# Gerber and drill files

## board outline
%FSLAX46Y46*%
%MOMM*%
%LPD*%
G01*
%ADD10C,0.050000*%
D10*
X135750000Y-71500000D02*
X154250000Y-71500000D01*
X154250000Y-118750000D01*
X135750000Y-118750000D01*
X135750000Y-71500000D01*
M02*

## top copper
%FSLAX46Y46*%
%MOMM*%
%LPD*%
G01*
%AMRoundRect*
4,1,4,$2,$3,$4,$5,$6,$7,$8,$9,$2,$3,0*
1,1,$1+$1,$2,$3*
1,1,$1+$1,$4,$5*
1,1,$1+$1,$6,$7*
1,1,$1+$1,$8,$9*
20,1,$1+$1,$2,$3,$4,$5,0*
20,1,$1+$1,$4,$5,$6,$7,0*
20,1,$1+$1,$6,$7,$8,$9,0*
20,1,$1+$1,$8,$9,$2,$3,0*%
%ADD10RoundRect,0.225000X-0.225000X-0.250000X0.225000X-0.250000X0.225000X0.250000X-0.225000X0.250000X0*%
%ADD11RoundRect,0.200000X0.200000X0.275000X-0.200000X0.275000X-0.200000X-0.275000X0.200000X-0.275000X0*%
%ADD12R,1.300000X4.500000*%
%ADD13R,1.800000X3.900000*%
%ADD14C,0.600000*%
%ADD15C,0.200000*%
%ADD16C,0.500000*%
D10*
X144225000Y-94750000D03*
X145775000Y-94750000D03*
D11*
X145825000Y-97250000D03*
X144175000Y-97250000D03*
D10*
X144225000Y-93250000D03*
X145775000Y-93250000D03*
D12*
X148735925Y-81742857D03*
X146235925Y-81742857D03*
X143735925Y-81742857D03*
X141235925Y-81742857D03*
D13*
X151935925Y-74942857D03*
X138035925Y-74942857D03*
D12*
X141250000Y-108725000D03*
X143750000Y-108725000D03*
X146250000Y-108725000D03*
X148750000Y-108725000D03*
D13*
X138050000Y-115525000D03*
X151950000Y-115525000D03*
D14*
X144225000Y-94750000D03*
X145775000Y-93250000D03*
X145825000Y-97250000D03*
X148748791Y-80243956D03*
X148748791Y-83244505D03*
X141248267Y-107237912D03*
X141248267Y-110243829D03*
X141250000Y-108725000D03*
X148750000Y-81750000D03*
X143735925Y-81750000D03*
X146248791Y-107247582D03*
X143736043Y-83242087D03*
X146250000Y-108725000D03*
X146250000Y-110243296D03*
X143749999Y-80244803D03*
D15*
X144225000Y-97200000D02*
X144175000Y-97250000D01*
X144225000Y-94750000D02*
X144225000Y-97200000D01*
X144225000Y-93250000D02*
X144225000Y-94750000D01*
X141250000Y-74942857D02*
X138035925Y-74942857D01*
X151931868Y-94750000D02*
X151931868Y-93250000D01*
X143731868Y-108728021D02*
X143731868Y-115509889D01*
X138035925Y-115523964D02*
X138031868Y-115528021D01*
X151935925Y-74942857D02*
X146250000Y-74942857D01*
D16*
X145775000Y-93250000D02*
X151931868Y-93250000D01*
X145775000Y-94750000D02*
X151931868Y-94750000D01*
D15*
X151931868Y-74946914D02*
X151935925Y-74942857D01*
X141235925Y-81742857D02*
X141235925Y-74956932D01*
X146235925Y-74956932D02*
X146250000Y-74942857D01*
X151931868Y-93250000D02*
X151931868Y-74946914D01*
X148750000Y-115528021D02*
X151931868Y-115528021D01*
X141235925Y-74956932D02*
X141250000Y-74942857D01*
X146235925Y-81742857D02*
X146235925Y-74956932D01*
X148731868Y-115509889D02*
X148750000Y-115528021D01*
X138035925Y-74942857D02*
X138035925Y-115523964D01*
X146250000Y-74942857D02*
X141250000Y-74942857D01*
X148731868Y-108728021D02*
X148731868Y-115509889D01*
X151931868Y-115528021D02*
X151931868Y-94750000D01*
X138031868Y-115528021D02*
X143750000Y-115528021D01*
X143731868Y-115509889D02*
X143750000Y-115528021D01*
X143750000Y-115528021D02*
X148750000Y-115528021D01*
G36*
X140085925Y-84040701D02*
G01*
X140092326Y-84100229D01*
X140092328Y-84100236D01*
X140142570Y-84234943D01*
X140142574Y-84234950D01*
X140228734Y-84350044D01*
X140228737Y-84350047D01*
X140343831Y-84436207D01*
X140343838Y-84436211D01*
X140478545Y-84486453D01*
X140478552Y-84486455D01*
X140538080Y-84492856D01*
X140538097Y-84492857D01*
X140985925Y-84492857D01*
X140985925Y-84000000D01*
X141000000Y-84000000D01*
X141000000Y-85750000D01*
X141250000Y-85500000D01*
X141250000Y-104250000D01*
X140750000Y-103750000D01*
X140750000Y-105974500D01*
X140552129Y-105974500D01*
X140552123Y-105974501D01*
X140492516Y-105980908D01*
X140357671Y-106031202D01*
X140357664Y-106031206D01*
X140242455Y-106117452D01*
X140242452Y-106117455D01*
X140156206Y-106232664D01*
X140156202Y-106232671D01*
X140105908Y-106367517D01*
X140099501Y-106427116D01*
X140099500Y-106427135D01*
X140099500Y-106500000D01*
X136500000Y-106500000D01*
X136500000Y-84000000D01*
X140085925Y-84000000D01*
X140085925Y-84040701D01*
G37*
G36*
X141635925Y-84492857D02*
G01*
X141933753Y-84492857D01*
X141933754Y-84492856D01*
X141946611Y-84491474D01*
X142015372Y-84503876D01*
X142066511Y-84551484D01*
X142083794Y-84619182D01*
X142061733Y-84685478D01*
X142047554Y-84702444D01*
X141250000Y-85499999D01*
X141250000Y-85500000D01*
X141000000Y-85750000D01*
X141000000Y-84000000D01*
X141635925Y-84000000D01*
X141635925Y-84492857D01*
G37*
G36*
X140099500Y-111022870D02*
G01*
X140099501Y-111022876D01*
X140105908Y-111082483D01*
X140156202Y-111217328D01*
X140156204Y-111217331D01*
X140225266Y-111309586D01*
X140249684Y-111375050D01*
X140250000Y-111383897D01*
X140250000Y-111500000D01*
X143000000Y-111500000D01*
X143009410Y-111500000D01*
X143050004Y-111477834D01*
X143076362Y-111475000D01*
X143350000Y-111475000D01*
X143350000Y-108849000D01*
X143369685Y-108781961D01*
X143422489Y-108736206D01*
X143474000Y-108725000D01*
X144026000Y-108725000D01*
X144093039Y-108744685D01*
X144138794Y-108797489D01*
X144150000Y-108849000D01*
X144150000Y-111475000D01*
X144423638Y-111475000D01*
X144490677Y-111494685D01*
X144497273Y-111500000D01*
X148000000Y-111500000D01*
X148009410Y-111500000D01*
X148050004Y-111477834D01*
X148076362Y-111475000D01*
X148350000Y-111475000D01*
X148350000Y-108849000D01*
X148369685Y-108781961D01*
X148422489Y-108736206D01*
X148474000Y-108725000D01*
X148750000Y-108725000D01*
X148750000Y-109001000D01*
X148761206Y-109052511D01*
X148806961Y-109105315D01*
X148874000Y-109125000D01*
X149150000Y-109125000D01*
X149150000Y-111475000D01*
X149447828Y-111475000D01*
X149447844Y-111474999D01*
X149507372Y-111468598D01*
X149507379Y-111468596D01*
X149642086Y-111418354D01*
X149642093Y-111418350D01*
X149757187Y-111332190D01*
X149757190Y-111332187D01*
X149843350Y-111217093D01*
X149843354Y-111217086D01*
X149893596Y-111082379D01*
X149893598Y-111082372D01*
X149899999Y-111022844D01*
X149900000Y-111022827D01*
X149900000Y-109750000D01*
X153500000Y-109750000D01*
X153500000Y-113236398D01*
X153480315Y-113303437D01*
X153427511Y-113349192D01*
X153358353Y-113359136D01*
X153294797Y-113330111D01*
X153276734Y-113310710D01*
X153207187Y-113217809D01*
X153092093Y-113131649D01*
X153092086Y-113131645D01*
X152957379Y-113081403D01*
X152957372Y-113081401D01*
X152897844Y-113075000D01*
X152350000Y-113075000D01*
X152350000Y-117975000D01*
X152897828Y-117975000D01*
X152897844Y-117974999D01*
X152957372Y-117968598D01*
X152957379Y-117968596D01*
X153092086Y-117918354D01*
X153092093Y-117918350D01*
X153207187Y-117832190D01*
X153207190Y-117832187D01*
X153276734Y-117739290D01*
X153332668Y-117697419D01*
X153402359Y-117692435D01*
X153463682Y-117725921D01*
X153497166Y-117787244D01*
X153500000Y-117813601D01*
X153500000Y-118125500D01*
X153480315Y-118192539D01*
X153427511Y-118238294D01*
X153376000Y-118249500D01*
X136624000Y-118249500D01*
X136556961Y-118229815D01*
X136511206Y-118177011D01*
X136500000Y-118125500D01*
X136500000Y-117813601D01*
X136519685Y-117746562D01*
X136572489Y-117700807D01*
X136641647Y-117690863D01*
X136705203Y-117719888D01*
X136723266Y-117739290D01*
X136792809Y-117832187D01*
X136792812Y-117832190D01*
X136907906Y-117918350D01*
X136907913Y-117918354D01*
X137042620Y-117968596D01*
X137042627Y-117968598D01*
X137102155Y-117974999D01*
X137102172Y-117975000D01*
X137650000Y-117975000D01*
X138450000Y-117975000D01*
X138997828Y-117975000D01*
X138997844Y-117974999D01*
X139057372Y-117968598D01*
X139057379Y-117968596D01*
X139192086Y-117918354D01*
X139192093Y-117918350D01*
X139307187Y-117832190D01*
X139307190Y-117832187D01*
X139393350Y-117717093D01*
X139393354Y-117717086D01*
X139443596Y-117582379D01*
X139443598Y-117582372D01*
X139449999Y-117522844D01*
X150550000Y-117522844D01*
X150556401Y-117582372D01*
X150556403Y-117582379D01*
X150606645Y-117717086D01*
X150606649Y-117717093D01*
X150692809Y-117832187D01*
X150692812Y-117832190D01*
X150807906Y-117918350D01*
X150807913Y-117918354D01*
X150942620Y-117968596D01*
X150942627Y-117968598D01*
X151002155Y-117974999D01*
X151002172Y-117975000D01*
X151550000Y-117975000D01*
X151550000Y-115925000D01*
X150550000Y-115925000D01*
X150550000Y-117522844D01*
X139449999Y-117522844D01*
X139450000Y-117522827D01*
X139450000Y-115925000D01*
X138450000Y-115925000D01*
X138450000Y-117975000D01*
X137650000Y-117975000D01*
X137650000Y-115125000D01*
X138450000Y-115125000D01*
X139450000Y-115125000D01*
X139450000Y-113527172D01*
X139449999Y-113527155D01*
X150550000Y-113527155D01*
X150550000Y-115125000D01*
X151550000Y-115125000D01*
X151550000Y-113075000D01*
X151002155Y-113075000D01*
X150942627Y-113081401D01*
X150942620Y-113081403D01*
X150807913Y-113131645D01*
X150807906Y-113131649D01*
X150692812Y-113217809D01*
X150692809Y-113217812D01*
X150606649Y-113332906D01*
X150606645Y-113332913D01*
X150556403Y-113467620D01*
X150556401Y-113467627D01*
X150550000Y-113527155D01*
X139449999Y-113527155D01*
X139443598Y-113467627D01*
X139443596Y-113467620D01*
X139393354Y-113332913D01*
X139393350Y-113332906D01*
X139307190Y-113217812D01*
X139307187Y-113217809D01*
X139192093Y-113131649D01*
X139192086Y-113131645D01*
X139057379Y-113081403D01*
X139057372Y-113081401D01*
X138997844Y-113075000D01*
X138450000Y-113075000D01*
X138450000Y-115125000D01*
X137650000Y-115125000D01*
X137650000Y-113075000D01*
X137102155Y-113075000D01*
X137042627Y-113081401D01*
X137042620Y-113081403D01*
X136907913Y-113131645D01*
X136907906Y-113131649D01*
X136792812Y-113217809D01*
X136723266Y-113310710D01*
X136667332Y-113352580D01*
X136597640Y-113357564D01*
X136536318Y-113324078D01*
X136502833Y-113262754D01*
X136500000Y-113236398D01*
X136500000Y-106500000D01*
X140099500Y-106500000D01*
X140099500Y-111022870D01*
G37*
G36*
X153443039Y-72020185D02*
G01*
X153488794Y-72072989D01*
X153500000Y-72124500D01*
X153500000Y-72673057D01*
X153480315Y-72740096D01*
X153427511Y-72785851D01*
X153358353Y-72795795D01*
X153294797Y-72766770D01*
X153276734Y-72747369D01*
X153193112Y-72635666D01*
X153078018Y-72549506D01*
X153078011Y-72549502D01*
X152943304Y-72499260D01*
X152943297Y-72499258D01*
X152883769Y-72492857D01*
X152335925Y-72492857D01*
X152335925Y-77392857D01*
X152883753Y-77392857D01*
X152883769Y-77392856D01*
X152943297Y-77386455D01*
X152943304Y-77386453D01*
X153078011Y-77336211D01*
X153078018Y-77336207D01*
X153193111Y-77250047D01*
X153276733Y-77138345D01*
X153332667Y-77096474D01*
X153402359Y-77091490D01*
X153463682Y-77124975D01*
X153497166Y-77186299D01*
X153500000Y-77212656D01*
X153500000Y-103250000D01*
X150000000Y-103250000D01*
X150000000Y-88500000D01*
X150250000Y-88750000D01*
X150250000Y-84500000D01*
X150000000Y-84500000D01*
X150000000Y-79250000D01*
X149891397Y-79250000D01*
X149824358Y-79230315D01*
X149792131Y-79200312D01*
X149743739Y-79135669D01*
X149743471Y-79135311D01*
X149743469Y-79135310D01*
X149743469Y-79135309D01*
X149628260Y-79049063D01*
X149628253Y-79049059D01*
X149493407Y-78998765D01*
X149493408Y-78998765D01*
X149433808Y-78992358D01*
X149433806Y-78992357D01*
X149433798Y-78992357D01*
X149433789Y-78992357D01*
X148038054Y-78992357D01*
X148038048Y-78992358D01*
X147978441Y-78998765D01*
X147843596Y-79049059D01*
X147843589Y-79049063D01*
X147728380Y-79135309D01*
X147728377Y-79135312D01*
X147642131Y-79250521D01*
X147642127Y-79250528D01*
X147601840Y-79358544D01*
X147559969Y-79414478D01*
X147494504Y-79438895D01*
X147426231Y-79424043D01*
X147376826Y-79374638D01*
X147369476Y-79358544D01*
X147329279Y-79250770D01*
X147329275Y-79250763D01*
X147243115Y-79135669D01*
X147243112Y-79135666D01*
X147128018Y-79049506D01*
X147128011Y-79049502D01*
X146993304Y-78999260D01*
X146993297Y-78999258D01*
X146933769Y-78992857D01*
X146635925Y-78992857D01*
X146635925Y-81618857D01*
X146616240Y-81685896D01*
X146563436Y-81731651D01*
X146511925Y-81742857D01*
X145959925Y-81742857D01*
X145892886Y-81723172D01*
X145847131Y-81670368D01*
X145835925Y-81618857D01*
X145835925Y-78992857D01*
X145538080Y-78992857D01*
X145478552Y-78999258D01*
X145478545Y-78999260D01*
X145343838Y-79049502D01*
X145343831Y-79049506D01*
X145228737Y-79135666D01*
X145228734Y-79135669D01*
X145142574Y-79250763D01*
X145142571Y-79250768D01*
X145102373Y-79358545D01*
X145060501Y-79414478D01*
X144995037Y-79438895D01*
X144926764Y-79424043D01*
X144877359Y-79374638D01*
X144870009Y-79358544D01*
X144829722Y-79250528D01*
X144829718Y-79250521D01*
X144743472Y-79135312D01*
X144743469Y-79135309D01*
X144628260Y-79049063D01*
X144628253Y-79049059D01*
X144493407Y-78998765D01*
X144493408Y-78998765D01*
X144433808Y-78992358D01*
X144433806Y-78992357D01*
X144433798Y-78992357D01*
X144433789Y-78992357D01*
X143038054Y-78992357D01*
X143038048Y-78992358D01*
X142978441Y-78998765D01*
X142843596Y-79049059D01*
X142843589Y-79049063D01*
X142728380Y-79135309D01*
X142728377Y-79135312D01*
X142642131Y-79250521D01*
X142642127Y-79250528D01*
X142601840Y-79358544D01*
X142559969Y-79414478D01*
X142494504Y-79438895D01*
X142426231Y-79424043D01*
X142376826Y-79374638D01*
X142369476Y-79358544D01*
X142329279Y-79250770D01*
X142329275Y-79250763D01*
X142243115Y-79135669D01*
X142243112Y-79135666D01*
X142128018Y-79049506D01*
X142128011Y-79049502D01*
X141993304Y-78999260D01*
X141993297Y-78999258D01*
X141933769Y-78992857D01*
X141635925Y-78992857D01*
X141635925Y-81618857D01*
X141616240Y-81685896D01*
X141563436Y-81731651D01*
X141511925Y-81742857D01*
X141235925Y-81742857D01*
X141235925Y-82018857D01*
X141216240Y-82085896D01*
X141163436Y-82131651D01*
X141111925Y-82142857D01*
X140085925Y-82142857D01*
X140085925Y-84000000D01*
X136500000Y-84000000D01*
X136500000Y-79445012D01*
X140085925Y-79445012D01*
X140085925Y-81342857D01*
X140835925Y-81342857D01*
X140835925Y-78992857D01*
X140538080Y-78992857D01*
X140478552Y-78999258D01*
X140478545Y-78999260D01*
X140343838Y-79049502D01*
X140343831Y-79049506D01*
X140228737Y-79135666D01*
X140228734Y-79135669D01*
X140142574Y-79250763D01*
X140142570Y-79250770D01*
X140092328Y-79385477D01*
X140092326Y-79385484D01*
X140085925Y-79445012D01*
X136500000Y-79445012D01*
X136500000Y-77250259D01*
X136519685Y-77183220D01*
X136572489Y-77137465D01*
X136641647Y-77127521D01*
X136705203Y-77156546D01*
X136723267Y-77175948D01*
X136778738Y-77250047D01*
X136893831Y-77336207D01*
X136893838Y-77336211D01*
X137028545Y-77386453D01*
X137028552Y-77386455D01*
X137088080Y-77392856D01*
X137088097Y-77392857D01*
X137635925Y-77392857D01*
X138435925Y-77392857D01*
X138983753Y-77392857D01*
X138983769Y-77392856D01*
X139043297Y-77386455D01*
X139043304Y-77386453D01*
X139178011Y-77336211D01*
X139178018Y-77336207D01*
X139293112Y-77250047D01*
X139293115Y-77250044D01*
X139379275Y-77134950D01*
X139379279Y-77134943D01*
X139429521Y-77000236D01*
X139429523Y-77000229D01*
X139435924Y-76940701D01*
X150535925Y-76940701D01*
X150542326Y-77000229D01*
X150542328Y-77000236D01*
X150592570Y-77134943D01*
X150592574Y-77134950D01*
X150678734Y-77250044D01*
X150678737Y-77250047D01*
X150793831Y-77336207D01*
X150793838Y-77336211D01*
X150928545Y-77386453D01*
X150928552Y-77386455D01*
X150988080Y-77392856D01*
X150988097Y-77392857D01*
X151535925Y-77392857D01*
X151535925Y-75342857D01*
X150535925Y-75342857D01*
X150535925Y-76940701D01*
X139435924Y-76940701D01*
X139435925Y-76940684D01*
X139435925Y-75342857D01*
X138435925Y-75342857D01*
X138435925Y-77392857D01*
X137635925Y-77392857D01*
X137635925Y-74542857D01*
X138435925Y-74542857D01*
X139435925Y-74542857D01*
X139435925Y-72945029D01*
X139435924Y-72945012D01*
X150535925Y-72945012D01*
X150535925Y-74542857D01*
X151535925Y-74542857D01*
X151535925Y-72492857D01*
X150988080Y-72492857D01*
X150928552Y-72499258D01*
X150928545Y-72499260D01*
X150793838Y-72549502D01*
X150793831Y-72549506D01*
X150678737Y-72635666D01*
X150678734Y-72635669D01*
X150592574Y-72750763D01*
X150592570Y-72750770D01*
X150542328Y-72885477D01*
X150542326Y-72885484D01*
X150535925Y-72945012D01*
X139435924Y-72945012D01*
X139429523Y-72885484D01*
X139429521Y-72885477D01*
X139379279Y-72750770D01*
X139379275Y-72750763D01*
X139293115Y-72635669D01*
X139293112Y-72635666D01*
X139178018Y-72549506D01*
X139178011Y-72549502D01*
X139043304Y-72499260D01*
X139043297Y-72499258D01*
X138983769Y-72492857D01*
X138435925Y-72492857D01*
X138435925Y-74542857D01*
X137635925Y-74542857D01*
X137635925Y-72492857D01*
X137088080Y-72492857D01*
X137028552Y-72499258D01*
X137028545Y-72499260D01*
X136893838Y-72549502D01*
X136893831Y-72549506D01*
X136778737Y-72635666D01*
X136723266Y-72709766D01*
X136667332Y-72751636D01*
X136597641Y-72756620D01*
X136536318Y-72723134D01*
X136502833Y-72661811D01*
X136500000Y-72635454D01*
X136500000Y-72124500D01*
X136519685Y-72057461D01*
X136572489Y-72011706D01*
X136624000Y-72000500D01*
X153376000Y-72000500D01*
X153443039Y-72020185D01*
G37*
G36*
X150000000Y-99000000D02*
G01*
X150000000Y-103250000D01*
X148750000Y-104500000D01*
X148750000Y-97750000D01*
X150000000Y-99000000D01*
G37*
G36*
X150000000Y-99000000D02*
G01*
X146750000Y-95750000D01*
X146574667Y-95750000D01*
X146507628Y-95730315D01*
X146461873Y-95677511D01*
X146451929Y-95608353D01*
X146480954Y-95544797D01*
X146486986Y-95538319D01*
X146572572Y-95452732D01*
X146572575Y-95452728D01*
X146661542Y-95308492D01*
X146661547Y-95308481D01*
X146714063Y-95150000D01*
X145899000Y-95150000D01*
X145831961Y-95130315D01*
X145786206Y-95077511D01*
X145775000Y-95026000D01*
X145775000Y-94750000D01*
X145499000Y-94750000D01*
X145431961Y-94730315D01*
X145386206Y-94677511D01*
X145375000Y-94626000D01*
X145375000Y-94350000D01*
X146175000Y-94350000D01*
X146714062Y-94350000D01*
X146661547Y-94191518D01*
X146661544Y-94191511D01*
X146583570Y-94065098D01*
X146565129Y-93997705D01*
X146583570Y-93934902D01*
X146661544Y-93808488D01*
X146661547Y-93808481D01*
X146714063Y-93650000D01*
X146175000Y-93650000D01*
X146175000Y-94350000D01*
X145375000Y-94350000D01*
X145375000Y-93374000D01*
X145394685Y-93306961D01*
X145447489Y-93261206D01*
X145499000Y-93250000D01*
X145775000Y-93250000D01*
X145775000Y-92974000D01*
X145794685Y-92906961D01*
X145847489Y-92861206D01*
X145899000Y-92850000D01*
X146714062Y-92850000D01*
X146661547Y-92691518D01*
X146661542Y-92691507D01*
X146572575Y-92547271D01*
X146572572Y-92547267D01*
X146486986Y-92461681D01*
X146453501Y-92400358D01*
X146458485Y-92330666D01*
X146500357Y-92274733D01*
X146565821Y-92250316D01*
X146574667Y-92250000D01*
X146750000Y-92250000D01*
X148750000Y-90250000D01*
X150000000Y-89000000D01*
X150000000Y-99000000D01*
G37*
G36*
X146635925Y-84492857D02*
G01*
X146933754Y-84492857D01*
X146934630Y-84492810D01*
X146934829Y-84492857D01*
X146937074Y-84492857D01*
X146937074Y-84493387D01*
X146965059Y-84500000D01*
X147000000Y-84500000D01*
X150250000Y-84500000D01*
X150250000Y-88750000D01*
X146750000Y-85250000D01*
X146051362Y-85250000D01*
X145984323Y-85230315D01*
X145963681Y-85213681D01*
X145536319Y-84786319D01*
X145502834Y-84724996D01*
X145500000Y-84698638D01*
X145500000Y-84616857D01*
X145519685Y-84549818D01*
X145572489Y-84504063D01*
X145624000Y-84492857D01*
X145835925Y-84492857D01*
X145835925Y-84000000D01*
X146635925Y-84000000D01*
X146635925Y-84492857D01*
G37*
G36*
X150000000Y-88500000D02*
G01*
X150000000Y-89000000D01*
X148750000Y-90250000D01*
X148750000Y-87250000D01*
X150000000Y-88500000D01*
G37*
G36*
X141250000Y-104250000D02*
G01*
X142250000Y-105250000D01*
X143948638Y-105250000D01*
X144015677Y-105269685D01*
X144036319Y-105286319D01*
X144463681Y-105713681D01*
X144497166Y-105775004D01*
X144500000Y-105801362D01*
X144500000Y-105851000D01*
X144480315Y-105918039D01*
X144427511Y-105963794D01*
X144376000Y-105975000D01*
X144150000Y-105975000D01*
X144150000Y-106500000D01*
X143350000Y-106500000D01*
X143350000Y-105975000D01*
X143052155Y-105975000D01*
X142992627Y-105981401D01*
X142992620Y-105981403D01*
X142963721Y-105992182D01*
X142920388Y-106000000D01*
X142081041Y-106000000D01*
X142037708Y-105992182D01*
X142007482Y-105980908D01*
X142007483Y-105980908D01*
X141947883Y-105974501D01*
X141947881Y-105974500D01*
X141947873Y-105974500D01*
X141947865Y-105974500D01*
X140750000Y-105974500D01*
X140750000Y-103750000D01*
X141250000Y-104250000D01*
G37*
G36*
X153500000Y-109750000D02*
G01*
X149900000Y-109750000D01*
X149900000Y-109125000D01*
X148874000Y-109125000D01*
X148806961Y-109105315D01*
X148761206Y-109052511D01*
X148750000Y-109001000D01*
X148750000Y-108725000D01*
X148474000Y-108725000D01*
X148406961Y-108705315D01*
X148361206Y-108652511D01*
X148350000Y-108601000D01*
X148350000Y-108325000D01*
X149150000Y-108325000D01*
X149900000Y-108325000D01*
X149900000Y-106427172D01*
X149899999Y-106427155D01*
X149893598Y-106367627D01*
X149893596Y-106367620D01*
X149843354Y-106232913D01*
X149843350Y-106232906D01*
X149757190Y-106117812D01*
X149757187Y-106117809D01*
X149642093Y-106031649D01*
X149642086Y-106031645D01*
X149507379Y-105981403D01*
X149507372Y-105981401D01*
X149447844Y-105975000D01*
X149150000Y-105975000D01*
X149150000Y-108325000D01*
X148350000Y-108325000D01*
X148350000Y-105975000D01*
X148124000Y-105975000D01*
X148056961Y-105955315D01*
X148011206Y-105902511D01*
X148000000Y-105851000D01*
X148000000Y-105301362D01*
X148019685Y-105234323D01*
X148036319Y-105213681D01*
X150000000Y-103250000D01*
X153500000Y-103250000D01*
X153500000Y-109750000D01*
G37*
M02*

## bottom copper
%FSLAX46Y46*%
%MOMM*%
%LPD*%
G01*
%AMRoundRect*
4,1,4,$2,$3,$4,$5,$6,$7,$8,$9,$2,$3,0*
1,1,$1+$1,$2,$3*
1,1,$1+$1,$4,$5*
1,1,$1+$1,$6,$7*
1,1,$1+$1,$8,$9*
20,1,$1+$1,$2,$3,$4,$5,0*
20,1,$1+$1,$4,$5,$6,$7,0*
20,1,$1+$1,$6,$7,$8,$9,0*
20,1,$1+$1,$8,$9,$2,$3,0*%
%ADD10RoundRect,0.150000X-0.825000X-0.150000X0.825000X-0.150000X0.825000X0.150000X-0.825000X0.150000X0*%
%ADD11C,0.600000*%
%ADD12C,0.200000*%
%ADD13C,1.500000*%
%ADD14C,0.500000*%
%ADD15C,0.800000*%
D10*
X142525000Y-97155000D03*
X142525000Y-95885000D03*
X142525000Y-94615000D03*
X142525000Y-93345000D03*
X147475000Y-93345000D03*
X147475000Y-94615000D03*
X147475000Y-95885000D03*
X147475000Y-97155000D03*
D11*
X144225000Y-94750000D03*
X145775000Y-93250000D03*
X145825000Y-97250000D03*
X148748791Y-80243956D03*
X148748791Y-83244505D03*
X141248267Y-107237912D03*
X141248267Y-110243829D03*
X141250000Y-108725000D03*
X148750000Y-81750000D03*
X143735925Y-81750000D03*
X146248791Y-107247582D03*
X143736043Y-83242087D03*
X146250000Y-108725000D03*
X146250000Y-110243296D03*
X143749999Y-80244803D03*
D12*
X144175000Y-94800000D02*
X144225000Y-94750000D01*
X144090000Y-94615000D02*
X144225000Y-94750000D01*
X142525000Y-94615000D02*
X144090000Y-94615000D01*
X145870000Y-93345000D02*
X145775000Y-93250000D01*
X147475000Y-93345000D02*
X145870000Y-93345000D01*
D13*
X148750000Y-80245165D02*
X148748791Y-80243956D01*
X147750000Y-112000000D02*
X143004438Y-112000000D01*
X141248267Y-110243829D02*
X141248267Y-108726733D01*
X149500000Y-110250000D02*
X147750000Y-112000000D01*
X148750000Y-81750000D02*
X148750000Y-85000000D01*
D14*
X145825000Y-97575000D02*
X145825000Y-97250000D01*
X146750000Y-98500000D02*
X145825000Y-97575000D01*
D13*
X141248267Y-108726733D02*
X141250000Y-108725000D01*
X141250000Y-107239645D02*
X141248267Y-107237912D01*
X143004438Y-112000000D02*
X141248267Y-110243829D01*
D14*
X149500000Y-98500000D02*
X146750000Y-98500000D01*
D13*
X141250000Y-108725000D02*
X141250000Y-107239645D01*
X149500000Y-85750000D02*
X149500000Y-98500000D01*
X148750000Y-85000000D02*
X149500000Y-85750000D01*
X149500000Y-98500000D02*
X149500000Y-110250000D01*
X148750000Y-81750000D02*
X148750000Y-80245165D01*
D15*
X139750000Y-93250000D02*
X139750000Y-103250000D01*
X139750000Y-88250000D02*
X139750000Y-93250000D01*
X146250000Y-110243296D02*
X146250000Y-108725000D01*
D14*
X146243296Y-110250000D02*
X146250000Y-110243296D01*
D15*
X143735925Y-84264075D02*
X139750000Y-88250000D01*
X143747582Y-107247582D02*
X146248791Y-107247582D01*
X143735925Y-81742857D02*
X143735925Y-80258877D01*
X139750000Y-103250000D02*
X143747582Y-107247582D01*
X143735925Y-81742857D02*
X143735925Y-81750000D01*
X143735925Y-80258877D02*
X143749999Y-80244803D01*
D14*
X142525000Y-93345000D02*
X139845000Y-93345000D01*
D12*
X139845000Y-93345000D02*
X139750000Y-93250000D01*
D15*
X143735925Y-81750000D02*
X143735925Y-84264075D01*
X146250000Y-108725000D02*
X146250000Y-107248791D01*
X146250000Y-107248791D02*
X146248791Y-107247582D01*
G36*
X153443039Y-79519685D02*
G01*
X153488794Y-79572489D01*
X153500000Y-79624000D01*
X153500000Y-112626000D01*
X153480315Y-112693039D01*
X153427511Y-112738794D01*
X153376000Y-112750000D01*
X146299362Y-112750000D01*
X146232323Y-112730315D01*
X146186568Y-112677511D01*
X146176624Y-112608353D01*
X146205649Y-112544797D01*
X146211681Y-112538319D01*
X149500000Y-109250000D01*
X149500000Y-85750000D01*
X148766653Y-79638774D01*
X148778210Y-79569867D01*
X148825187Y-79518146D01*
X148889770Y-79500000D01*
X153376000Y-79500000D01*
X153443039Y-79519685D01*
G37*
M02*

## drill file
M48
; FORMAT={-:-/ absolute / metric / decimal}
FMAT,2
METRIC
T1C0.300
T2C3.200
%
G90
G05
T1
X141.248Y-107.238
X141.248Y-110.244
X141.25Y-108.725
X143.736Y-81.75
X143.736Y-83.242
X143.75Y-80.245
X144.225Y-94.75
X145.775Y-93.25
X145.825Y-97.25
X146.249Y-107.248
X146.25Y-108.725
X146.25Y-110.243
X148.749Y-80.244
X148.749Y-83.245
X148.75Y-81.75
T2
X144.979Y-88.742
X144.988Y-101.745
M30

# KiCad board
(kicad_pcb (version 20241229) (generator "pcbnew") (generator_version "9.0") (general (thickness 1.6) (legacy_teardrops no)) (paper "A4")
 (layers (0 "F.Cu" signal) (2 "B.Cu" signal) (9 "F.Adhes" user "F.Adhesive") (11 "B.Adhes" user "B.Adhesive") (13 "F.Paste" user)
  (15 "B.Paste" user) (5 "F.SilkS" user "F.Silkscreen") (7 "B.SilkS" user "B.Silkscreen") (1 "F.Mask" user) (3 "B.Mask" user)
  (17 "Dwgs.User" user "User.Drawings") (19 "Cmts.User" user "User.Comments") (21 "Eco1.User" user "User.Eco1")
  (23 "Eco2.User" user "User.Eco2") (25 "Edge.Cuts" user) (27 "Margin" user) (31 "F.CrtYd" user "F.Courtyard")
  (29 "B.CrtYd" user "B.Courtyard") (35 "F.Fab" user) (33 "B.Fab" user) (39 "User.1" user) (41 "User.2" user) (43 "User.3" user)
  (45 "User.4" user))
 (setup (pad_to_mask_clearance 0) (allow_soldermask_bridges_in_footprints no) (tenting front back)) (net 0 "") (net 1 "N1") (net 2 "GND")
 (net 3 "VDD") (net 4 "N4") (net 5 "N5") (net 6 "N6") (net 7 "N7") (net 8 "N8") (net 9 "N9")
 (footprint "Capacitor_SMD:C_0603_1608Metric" (layer "F.Cu") (at 145 94.75)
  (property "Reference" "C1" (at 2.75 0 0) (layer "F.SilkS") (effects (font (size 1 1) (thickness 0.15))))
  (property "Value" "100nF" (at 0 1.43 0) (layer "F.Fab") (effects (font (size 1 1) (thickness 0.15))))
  (pad "1" smd roundrect (at -0.775 0) (size 0.9 0.95) (layers "F.Cu" "F.Mask" "F.Paste") (roundrect_rratio 0.25) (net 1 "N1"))
  (pad "2" smd roundrect (at 0.775 0) (size 0.9 0.95) (layers "F.Cu" "F.Mask" "F.Paste") (roundrect_rratio 0.25) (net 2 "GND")))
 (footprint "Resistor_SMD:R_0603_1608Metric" (layer "F.Cu") (at 145 97.25 180)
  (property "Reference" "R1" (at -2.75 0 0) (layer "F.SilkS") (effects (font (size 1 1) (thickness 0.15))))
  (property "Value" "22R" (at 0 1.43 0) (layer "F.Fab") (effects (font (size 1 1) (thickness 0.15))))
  (pad "1" smd roundrect (at -0.825 0 180) (size 0.8 0.95) (layers "F.Cu" "F.Mask" "F.Paste") (roundrect_rratio 0.25) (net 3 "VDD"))
  (pad "2" smd roundrect (at 0.825 0 180) (size 0.8 0.95) (layers "F.Cu" "F.Mask" "F.Paste") (roundrect_rratio 0.25) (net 1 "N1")))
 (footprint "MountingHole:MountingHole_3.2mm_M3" (layer "F.Cu") (at 144.988461 101.744505)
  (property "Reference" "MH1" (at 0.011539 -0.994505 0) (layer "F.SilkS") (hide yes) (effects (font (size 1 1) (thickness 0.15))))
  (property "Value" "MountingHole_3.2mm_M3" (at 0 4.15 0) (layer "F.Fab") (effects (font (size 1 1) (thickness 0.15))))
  (pad "" np_thru_hole circle (at 0 0) (size 3.2 3.2) (drill 3.2) (layers "*.Cu" "*.Mask")))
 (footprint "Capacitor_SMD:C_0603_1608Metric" (layer "F.Cu") (at 145 93.25)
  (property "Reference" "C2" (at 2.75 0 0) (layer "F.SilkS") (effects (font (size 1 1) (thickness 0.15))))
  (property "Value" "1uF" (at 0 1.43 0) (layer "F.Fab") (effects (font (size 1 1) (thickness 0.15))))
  (pad "1" smd roundrect (at -0.775 0) (size 0.9 0.95) (layers "F.Cu" "F.Mask" "F.Paste") (roundrect_rratio 0.25) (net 1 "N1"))
  (pad "2" smd roundrect (at 0.775 0) (size 0.9 0.95) (layers "F.Cu" "F.Mask" "F.Paste") (roundrect_rratio 0.25) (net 2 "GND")))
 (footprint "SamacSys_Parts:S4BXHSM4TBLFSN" (layer "F.Cu") (at 144.985925 77.467857 180)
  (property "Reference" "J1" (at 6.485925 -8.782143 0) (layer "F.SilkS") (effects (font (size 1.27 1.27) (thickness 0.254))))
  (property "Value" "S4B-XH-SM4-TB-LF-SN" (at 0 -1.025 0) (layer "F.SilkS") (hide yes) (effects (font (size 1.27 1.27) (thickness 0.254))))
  (pad "1" smd rect (at -3.75 -4.275 180) (size 1.3 4.5) (layers "F.Cu" "F.Mask" "F.Paste") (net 3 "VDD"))
  (pad "2" smd rect (at -1.25 -4.275 180) (size 1.3 4.5) (layers "F.Cu" "F.Mask" "F.Paste") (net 2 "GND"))
  (pad "3" smd rect (at 1.25 -4.275 180) (size 1.3 4.5) (layers "F.Cu" "F.Mask" "F.Paste") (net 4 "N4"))
  (pad "4" smd rect (at 3.75 -4.275 180) (size 1.3 4.5) (layers "F.Cu" "F.Mask" "F.Paste") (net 2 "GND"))
  (pad "MP1" smd rect (at -6.95 2.525 180) (size 1.8 3.9) (layers "F.Cu" "F.Mask" "F.Paste") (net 2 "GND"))
  (pad "MP2" smd rect (at 6.95 2.525 180) (size 1.8 3.9) (layers "F.Cu" "F.Mask" "F.Paste") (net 2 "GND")))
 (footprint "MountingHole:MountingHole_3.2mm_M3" (layer "F.Cu") (at 144.978529 88.742349)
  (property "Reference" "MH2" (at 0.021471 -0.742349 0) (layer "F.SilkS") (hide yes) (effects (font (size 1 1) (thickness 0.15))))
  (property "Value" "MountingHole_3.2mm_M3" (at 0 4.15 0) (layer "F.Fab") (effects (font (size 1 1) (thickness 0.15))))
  (pad "" np_thru_hole circle (at 0 0) (size 3.2 3.2) (drill 3.2) (layers "*.Cu" "*.Mask")))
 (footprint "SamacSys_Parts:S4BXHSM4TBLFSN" (layer "F.Cu") (at 145 113)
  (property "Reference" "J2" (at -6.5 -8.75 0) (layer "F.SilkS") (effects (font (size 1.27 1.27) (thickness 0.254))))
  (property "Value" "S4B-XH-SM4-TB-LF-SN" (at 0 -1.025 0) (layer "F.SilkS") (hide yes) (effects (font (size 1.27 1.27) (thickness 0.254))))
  (pad "1" smd rect (at -3.75 -4.275) (size 1.3 4.5) (layers "F.Cu" "F.Mask" "F.Paste") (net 3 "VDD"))
  (pad "2" smd rect (at -1.25 -4.275) (size 1.3 4.5) (layers "F.Cu" "F.Mask" "F.Paste") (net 2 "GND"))
  (pad "3" smd rect (at 1.25 -4.275) (size 1.3 4.5) (layers "F.Cu" "F.Mask" "F.Paste") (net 4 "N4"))
  (pad "4" smd rect (at 3.75 -4.275) (size 1.3 4.5) (layers "F.Cu" "F.Mask" "F.Paste") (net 2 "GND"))
  (pad "MP1" smd rect (at -6.95 2.525) (size 1.8 3.9) (layers "F.Cu" "F.Mask" "F.Paste") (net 2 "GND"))
  (pad "MP2" smd rect (at 6.95 2.525) (size 1.8 3.9) (layers "F.Cu" "F.Mask" "F.Paste") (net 2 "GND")))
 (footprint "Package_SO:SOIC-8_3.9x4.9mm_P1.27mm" (layer "B.Cu") (at 145 95.25)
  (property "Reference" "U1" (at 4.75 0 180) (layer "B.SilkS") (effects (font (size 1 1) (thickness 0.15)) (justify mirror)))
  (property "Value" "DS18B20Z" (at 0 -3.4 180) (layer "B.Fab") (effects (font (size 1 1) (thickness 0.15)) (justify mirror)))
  (pad "1" smd roundrect (at -2.475 1.905) (size 1.95 0.6) (layers "B.Cu" "B.Mask" "B.Paste") (roundrect_rratio 0.25) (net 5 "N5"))
  (pad "2" smd roundrect (at -2.475 0.635) (size 1.95 0.6) (layers "B.Cu" "B.Mask" "B.Paste") (roundrect_rratio 0.25) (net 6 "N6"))
  (pad "3" smd roundrect (at -2.475 -0.635) (size 1.95 0.6) (layers "B.Cu" "B.Mask" "B.Paste") (roundrect_rratio 0.25) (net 1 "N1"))
  (pad "4" smd roundrect (at -2.475 -1.905) (size 1.95 0.6) (layers "B.Cu" "B.Mask" "B.Paste") (roundrect_rratio 0.25) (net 4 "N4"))
  (pad "5" smd roundrect (at 2.475 -1.905) (size 1.95 0.6) (layers "B.Cu" "B.Mask" "B.Paste") (roundrect_rratio 0.25) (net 2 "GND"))
  (pad "6" smd roundrect (at 2.475 -0.635) (size 1.95 0.6) (layers "B.Cu" "B.Mask" "B.Paste") (roundrect_rratio 0.25) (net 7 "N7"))
  (pad "7" smd roundrect (at 2.475 0.635) (size 1.95 0.6) (layers "B.Cu" "B.Mask" "B.Paste") (roundrect_rratio 0.25) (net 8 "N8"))
  (pad "8" smd roundrect (at 2.475 1.905) (size 1.95 0.6) (layers "B.Cu" "B.Mask" "B.Paste") (roundrect_rratio 0.25) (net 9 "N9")))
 (gr_rect (start 135.75 71.5) (end 154.25 118.75) (stroke (width 0.05) (type default)) (fill no) (layer "Edge.Cuts"))
 (segment (start 144.225 97.2) (end 144.175 97.25) (width 0.2) (layer "F.Cu") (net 1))
 (segment (start 144.225 94.75) (end 144.225 97.2) (width 0.2) (layer "F.Cu") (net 1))
 (segment (start 144.225 93.25) (end 144.225 94.75) (width 0.2) (layer "F.Cu") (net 1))
 (via (at 144.225 94.75) (size 0.6) (drill 0.3) (layers "F.Cu" "B.Cu") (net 1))
 (segment (start 144.175 94.8) (end 144.225 94.75) (width 0.2) (layer "B.Cu") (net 1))
 (segment (start 144.09 94.615) (end 144.225 94.75) (width 0.2) (layer "B.Cu") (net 1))
 (segment (start 142.525 94.615) (end 144.09 94.615) (width 0.2) (layer "B.Cu") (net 1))
 (segment (start 141.25 74.942857) (end 138.035925 74.942857) (width 0.2) (layer "F.Cu") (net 2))
 (segment (start 151.931868 94.75) (end 151.931868 93.25) (width 0.2) (layer "F.Cu") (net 2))
 (segment (start 143.731868 108.728021) (end 143.731868 115.509889) (width 0.2) (layer "F.Cu") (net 2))
 (segment (start 138.035925 115.523964) (end 138.031868 115.528021) (width 0.2) (layer "F.Cu") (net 2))
 (segment (start 151.935925 74.942857) (end 146.25 74.942857) (width 0.2) (layer "F.Cu") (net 2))
 (segment (start 145.775 93.25) (end 151.931868 93.25) (width 0.5) (layer "F.Cu") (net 2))
 (segment (start 145.775 94.75) (end 151.931868 94.75) (width 0.5) (layer "F.Cu") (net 2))
 (segment (start 151.931868 74.946914) (end 151.935925 74.942857) (width 0.2) (layer "F.Cu") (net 2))
 (segment (start 141.235925 81.742857) (end 141.235925 74.956932) (width 0.2) (layer "F.Cu") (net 2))
 (segment (start 146.235925 74.956932) (end 146.25 74.942857) (width 0.2) (layer "F.Cu") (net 2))
 (segment (start 151.931868 93.25) (end 151.931868 74.946914) (width 0.2) (layer "F.Cu") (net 2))
 (segment (start 148.75 115.528021) (end 151.931868 115.528021) (width 0.2) (layer "F.Cu") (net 2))
 (segment (start 141.235925 74.956932) (end 141.25 74.942857) (width 0.2) (layer "F.Cu") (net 2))
 (segment (start 146.235925 81.742857) (end 146.235925 74.956932) (width 0.2) (layer "F.Cu") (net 2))
 (segment (start 148.731868 115.509889) (end 148.75 115.528021) (width 0.2) (layer "F.Cu") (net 2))
 (segment (start 138.035925 74.942857) (end 138.035925 115.523964) (width 0.2) (layer "F.Cu") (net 2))
 (segment (start 146.25 74.942857) (end 141.25 74.942857) (width 0.2) (layer "F.Cu") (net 2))
 (segment (start 148.731868 108.728021) (end 148.731868 115.509889) (width 0.2) (layer "F.Cu") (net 2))
 (segment (start 151.931868 115.528021) (end 151.931868 94.75) (width 0.2) (layer "F.Cu") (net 2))
 (segment (start 138.031868 115.528021) (end 143.75 115.528021) (width 0.2) (layer "F.Cu") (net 2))
 (segment (start 143.731868 115.509889) (end 143.75 115.528021) (width 0.2) (layer "F.Cu") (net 2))
 (segment (start 143.75 115.528021) (end 148.75 115.528021) (width 0.2) (layer "F.Cu") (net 2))
 (via (at 145.775 93.25) (size 0.6) (drill 0.3) (layers "F.Cu" "B.Cu") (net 2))
 (segment (start 145.87 93.345) (end 145.775 93.25) (width 0.2) (layer "B.Cu") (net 2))
 (segment (start 147.475 93.345) (end 145.87 93.345) (width 0.2) (layer "B.Cu") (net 2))
 (via (at 145.825 97.25) (size 0.6) (drill 0.3) (layers "F.Cu" "B.Cu") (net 3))
 (via (at 148.748791 80.243956) (size 0.6) (drill 0.3) (layers "F.Cu" "B.Cu") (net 3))
 (via (at 148.748791 83.244505) (size 0.6) (drill 0.3) (layers "F.Cu" "B.Cu") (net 3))
 (via (at 141.248267 107.237912) (size 0.6) (drill 0.3) (layers "F.Cu" "B.Cu") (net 3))
 (via (at 141.248267 110.243829) (size 0.6) (drill 0.3) (layers "F.Cu" "B.Cu") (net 3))
 (via (at 141.25 108.725) (size 0.6) (drill 0.3) (layers "F.Cu" "B.Cu") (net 3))
 (via (at 148.75 81.75) (size 0.6) (drill 0.3) (layers "F.Cu" "B.Cu") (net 3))
 (segment (start 148.75 80.245165) (end 148.748791 80.243956) (width 1.5) (layer "B.Cu") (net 3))
 (segment (start 147.75 112) (end 143.004438 112) (width 1.5) (layer "B.Cu") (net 3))
 (segment (start 141.248267 110.243829) (end 141.248267 108.726733) (width 1.5) (layer "B.Cu") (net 3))
 (segment (start 149.5 110.25) (end 147.75 112) (width 1.5) (layer "B.Cu") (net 3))
 (segment (start 148.75 81.75) (end 148.75 85) (width 1.5) (layer "B.Cu") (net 3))
 (segment (start 145.825 97.575) (end 145.825 97.25) (width 0.5) (layer "B.Cu") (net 3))
 (segment (start 146.75 98.5) (end 145.825 97.575) (width 0.5) (layer "B.Cu") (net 3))
 (segment (start 141.248267 108.726733) (end 141.25 108.725) (width 1.5) (layer "B.Cu") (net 3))
 (segment (start 141.25 107.239645) (end 141.248267 107.237912) (width 1.5) (layer "B.Cu") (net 3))
 (segment (start 143.004438 112) (end 141.248267 110.243829) (width 1.5) (layer "B.Cu") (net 3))
 (segment (start 149.5 98.5) (end 146.75 98.5) (width 0.5) (layer "B.Cu") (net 3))
 (segment (start 141.25 108.725) (end 141.25 107.239645) (width 1.5) (layer "B.Cu") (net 3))
 (segment (start 149.5 85.75) (end 149.5 98.5) (width 1.5) (layer "B.Cu") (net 3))
 (segment (start 148.75 85) (end 149.5 85.75) (width 1.5) (layer "B.Cu") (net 3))
 (segment (start 149.5 98.5) (end 149.5 110.25) (width 1.5) (layer "B.Cu") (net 3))
 (segment (start 148.75 81.75) (end 148.75 80.245165) (width 1.5) (layer "B.Cu") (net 3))
 (via (at 143.735925 81.75) (size 0.6) (drill 0.3) (layers "F.Cu" "B.Cu") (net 4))
 (via (at 146.248791 107.247582) (size 0.6) (drill 0.3) (layers "F.Cu" "B.Cu") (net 4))
 (via (at 143.736043 83.242087) (size 0.6) (drill 0.3) (layers "F.Cu" "B.Cu") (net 4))
 (via (at 146.25 108.725) (size 0.6) (drill 0.3) (layers "F.Cu" "B.Cu") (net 4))
 (via (at 146.25 110.243296) (size 0.6) (drill 0.3) (layers "F.Cu" "B.Cu") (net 4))
 (via (at 143.749999 80.244803) (size 0.6) (drill 0.3) (layers "F.Cu" "B.Cu") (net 4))
 (segment (start 139.75 93.25) (end 139.75 103.25) (width 0.8) (layer "B.Cu") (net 4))
 (segment (start 139.75 88.25) (end 139.75 93.25) (width 0.8) (layer "B.Cu") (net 4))
 (segment (start 146.25 110.243296) (end 146.25 108.725) (width 0.8) (layer "B.Cu") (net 4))
 (segment (start 146.243296 110.25) (end 146.25 110.243296) (width 0.5) (layer "B.Cu") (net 4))
 (segment (start 143.735925 84.264075) (end 139.75 88.25) (width 0.8) (layer "B.Cu") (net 4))
 (segment (start 143.747582 107.247582) (end 146.248791 107.247582) (width 0.8) (layer "B.Cu") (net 4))
 (segment (start 143.735925 81.742857) (end 143.735925 80.258877) (width 0.8) (layer "B.Cu") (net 4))
 (segment (start 139.75 103.25) (end 143.747582 107.247582) (width 0.8) (layer "B.Cu") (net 4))
 (segment (start 143.735925 81.742857) (end 143.735925 81.75) (width 0.8) (layer "B.Cu") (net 4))
 (segment (start 143.735925 80.258877) (end 143.749999 80.244803) (width 0.8) (layer "B.Cu") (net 4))
 (segment (start 142.525 93.345) (end 139.845 93.345) (width 0.5) (layer "B.Cu") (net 4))
 (segment (start 139.845 93.345) (end 139.75 93.25) (width 0.2) (layer "B.Cu") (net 4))
 (segment (start 143.735925 81.75) (end 143.735925 84.264075) (width 0.8) (layer "B.Cu") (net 4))
 (segment (start 146.25 108.725) (end 146.25 107.248791) (width 0.8) (layer "B.Cu") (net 4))
 (segment (start 146.25 107.248791) (end 146.248791 107.247582) (width 0.8) (layer "B.Cu") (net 4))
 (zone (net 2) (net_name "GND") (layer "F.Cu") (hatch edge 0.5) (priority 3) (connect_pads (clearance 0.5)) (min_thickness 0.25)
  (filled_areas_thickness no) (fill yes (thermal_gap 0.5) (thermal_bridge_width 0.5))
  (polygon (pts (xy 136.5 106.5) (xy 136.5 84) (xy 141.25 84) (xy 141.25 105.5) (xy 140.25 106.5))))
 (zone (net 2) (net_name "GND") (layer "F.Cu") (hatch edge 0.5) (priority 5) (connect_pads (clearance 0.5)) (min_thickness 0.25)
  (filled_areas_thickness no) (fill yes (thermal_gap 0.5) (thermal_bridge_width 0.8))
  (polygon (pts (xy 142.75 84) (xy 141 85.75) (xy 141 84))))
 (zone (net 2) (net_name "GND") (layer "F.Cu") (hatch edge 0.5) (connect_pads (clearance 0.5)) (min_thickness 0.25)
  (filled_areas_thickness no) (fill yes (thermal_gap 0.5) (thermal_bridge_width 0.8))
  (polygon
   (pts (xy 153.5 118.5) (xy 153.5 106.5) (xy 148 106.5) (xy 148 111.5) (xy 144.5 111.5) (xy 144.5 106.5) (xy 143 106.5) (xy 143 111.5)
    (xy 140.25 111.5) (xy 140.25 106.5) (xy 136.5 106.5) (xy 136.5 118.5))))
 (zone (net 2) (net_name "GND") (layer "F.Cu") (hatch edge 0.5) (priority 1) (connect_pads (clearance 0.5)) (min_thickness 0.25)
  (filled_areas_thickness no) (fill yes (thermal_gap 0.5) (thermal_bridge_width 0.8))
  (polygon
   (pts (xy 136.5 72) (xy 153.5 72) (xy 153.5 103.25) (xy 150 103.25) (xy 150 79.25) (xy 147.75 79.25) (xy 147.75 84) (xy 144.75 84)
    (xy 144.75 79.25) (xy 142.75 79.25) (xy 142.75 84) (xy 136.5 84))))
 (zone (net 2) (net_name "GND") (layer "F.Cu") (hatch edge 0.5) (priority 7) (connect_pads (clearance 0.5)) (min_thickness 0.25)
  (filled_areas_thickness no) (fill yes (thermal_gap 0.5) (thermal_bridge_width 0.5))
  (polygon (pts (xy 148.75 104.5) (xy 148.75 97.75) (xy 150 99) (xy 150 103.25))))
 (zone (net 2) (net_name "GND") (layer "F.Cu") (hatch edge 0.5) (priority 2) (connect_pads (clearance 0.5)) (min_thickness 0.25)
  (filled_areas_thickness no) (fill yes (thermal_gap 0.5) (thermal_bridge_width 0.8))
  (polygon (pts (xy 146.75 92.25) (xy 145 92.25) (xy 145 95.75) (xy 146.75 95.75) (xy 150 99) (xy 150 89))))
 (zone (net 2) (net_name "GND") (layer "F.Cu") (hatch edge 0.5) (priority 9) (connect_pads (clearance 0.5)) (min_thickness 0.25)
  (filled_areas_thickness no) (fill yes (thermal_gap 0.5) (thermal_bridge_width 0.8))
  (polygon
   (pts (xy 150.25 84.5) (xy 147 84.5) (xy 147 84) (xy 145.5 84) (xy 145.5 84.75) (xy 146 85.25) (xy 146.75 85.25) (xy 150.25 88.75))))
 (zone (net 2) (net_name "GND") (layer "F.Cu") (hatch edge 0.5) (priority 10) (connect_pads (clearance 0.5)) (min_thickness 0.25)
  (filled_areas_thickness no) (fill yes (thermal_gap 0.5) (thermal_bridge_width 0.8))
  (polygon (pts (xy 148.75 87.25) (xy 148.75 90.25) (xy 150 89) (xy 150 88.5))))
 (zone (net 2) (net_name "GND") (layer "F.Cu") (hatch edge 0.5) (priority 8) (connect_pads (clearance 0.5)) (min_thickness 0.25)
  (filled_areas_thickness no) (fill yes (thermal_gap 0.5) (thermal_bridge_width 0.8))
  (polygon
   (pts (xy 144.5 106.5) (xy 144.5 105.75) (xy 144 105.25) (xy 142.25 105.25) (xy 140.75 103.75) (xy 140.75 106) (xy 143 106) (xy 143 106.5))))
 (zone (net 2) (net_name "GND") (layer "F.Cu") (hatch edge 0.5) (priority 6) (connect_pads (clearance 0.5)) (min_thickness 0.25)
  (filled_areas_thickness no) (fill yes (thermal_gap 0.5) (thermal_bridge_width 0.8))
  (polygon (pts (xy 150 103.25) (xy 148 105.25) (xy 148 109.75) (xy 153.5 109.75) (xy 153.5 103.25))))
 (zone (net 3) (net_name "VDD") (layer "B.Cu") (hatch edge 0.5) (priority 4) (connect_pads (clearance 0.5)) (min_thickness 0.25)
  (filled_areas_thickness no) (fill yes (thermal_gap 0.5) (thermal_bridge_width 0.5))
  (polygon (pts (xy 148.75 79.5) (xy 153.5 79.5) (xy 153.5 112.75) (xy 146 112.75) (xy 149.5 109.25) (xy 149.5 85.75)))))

